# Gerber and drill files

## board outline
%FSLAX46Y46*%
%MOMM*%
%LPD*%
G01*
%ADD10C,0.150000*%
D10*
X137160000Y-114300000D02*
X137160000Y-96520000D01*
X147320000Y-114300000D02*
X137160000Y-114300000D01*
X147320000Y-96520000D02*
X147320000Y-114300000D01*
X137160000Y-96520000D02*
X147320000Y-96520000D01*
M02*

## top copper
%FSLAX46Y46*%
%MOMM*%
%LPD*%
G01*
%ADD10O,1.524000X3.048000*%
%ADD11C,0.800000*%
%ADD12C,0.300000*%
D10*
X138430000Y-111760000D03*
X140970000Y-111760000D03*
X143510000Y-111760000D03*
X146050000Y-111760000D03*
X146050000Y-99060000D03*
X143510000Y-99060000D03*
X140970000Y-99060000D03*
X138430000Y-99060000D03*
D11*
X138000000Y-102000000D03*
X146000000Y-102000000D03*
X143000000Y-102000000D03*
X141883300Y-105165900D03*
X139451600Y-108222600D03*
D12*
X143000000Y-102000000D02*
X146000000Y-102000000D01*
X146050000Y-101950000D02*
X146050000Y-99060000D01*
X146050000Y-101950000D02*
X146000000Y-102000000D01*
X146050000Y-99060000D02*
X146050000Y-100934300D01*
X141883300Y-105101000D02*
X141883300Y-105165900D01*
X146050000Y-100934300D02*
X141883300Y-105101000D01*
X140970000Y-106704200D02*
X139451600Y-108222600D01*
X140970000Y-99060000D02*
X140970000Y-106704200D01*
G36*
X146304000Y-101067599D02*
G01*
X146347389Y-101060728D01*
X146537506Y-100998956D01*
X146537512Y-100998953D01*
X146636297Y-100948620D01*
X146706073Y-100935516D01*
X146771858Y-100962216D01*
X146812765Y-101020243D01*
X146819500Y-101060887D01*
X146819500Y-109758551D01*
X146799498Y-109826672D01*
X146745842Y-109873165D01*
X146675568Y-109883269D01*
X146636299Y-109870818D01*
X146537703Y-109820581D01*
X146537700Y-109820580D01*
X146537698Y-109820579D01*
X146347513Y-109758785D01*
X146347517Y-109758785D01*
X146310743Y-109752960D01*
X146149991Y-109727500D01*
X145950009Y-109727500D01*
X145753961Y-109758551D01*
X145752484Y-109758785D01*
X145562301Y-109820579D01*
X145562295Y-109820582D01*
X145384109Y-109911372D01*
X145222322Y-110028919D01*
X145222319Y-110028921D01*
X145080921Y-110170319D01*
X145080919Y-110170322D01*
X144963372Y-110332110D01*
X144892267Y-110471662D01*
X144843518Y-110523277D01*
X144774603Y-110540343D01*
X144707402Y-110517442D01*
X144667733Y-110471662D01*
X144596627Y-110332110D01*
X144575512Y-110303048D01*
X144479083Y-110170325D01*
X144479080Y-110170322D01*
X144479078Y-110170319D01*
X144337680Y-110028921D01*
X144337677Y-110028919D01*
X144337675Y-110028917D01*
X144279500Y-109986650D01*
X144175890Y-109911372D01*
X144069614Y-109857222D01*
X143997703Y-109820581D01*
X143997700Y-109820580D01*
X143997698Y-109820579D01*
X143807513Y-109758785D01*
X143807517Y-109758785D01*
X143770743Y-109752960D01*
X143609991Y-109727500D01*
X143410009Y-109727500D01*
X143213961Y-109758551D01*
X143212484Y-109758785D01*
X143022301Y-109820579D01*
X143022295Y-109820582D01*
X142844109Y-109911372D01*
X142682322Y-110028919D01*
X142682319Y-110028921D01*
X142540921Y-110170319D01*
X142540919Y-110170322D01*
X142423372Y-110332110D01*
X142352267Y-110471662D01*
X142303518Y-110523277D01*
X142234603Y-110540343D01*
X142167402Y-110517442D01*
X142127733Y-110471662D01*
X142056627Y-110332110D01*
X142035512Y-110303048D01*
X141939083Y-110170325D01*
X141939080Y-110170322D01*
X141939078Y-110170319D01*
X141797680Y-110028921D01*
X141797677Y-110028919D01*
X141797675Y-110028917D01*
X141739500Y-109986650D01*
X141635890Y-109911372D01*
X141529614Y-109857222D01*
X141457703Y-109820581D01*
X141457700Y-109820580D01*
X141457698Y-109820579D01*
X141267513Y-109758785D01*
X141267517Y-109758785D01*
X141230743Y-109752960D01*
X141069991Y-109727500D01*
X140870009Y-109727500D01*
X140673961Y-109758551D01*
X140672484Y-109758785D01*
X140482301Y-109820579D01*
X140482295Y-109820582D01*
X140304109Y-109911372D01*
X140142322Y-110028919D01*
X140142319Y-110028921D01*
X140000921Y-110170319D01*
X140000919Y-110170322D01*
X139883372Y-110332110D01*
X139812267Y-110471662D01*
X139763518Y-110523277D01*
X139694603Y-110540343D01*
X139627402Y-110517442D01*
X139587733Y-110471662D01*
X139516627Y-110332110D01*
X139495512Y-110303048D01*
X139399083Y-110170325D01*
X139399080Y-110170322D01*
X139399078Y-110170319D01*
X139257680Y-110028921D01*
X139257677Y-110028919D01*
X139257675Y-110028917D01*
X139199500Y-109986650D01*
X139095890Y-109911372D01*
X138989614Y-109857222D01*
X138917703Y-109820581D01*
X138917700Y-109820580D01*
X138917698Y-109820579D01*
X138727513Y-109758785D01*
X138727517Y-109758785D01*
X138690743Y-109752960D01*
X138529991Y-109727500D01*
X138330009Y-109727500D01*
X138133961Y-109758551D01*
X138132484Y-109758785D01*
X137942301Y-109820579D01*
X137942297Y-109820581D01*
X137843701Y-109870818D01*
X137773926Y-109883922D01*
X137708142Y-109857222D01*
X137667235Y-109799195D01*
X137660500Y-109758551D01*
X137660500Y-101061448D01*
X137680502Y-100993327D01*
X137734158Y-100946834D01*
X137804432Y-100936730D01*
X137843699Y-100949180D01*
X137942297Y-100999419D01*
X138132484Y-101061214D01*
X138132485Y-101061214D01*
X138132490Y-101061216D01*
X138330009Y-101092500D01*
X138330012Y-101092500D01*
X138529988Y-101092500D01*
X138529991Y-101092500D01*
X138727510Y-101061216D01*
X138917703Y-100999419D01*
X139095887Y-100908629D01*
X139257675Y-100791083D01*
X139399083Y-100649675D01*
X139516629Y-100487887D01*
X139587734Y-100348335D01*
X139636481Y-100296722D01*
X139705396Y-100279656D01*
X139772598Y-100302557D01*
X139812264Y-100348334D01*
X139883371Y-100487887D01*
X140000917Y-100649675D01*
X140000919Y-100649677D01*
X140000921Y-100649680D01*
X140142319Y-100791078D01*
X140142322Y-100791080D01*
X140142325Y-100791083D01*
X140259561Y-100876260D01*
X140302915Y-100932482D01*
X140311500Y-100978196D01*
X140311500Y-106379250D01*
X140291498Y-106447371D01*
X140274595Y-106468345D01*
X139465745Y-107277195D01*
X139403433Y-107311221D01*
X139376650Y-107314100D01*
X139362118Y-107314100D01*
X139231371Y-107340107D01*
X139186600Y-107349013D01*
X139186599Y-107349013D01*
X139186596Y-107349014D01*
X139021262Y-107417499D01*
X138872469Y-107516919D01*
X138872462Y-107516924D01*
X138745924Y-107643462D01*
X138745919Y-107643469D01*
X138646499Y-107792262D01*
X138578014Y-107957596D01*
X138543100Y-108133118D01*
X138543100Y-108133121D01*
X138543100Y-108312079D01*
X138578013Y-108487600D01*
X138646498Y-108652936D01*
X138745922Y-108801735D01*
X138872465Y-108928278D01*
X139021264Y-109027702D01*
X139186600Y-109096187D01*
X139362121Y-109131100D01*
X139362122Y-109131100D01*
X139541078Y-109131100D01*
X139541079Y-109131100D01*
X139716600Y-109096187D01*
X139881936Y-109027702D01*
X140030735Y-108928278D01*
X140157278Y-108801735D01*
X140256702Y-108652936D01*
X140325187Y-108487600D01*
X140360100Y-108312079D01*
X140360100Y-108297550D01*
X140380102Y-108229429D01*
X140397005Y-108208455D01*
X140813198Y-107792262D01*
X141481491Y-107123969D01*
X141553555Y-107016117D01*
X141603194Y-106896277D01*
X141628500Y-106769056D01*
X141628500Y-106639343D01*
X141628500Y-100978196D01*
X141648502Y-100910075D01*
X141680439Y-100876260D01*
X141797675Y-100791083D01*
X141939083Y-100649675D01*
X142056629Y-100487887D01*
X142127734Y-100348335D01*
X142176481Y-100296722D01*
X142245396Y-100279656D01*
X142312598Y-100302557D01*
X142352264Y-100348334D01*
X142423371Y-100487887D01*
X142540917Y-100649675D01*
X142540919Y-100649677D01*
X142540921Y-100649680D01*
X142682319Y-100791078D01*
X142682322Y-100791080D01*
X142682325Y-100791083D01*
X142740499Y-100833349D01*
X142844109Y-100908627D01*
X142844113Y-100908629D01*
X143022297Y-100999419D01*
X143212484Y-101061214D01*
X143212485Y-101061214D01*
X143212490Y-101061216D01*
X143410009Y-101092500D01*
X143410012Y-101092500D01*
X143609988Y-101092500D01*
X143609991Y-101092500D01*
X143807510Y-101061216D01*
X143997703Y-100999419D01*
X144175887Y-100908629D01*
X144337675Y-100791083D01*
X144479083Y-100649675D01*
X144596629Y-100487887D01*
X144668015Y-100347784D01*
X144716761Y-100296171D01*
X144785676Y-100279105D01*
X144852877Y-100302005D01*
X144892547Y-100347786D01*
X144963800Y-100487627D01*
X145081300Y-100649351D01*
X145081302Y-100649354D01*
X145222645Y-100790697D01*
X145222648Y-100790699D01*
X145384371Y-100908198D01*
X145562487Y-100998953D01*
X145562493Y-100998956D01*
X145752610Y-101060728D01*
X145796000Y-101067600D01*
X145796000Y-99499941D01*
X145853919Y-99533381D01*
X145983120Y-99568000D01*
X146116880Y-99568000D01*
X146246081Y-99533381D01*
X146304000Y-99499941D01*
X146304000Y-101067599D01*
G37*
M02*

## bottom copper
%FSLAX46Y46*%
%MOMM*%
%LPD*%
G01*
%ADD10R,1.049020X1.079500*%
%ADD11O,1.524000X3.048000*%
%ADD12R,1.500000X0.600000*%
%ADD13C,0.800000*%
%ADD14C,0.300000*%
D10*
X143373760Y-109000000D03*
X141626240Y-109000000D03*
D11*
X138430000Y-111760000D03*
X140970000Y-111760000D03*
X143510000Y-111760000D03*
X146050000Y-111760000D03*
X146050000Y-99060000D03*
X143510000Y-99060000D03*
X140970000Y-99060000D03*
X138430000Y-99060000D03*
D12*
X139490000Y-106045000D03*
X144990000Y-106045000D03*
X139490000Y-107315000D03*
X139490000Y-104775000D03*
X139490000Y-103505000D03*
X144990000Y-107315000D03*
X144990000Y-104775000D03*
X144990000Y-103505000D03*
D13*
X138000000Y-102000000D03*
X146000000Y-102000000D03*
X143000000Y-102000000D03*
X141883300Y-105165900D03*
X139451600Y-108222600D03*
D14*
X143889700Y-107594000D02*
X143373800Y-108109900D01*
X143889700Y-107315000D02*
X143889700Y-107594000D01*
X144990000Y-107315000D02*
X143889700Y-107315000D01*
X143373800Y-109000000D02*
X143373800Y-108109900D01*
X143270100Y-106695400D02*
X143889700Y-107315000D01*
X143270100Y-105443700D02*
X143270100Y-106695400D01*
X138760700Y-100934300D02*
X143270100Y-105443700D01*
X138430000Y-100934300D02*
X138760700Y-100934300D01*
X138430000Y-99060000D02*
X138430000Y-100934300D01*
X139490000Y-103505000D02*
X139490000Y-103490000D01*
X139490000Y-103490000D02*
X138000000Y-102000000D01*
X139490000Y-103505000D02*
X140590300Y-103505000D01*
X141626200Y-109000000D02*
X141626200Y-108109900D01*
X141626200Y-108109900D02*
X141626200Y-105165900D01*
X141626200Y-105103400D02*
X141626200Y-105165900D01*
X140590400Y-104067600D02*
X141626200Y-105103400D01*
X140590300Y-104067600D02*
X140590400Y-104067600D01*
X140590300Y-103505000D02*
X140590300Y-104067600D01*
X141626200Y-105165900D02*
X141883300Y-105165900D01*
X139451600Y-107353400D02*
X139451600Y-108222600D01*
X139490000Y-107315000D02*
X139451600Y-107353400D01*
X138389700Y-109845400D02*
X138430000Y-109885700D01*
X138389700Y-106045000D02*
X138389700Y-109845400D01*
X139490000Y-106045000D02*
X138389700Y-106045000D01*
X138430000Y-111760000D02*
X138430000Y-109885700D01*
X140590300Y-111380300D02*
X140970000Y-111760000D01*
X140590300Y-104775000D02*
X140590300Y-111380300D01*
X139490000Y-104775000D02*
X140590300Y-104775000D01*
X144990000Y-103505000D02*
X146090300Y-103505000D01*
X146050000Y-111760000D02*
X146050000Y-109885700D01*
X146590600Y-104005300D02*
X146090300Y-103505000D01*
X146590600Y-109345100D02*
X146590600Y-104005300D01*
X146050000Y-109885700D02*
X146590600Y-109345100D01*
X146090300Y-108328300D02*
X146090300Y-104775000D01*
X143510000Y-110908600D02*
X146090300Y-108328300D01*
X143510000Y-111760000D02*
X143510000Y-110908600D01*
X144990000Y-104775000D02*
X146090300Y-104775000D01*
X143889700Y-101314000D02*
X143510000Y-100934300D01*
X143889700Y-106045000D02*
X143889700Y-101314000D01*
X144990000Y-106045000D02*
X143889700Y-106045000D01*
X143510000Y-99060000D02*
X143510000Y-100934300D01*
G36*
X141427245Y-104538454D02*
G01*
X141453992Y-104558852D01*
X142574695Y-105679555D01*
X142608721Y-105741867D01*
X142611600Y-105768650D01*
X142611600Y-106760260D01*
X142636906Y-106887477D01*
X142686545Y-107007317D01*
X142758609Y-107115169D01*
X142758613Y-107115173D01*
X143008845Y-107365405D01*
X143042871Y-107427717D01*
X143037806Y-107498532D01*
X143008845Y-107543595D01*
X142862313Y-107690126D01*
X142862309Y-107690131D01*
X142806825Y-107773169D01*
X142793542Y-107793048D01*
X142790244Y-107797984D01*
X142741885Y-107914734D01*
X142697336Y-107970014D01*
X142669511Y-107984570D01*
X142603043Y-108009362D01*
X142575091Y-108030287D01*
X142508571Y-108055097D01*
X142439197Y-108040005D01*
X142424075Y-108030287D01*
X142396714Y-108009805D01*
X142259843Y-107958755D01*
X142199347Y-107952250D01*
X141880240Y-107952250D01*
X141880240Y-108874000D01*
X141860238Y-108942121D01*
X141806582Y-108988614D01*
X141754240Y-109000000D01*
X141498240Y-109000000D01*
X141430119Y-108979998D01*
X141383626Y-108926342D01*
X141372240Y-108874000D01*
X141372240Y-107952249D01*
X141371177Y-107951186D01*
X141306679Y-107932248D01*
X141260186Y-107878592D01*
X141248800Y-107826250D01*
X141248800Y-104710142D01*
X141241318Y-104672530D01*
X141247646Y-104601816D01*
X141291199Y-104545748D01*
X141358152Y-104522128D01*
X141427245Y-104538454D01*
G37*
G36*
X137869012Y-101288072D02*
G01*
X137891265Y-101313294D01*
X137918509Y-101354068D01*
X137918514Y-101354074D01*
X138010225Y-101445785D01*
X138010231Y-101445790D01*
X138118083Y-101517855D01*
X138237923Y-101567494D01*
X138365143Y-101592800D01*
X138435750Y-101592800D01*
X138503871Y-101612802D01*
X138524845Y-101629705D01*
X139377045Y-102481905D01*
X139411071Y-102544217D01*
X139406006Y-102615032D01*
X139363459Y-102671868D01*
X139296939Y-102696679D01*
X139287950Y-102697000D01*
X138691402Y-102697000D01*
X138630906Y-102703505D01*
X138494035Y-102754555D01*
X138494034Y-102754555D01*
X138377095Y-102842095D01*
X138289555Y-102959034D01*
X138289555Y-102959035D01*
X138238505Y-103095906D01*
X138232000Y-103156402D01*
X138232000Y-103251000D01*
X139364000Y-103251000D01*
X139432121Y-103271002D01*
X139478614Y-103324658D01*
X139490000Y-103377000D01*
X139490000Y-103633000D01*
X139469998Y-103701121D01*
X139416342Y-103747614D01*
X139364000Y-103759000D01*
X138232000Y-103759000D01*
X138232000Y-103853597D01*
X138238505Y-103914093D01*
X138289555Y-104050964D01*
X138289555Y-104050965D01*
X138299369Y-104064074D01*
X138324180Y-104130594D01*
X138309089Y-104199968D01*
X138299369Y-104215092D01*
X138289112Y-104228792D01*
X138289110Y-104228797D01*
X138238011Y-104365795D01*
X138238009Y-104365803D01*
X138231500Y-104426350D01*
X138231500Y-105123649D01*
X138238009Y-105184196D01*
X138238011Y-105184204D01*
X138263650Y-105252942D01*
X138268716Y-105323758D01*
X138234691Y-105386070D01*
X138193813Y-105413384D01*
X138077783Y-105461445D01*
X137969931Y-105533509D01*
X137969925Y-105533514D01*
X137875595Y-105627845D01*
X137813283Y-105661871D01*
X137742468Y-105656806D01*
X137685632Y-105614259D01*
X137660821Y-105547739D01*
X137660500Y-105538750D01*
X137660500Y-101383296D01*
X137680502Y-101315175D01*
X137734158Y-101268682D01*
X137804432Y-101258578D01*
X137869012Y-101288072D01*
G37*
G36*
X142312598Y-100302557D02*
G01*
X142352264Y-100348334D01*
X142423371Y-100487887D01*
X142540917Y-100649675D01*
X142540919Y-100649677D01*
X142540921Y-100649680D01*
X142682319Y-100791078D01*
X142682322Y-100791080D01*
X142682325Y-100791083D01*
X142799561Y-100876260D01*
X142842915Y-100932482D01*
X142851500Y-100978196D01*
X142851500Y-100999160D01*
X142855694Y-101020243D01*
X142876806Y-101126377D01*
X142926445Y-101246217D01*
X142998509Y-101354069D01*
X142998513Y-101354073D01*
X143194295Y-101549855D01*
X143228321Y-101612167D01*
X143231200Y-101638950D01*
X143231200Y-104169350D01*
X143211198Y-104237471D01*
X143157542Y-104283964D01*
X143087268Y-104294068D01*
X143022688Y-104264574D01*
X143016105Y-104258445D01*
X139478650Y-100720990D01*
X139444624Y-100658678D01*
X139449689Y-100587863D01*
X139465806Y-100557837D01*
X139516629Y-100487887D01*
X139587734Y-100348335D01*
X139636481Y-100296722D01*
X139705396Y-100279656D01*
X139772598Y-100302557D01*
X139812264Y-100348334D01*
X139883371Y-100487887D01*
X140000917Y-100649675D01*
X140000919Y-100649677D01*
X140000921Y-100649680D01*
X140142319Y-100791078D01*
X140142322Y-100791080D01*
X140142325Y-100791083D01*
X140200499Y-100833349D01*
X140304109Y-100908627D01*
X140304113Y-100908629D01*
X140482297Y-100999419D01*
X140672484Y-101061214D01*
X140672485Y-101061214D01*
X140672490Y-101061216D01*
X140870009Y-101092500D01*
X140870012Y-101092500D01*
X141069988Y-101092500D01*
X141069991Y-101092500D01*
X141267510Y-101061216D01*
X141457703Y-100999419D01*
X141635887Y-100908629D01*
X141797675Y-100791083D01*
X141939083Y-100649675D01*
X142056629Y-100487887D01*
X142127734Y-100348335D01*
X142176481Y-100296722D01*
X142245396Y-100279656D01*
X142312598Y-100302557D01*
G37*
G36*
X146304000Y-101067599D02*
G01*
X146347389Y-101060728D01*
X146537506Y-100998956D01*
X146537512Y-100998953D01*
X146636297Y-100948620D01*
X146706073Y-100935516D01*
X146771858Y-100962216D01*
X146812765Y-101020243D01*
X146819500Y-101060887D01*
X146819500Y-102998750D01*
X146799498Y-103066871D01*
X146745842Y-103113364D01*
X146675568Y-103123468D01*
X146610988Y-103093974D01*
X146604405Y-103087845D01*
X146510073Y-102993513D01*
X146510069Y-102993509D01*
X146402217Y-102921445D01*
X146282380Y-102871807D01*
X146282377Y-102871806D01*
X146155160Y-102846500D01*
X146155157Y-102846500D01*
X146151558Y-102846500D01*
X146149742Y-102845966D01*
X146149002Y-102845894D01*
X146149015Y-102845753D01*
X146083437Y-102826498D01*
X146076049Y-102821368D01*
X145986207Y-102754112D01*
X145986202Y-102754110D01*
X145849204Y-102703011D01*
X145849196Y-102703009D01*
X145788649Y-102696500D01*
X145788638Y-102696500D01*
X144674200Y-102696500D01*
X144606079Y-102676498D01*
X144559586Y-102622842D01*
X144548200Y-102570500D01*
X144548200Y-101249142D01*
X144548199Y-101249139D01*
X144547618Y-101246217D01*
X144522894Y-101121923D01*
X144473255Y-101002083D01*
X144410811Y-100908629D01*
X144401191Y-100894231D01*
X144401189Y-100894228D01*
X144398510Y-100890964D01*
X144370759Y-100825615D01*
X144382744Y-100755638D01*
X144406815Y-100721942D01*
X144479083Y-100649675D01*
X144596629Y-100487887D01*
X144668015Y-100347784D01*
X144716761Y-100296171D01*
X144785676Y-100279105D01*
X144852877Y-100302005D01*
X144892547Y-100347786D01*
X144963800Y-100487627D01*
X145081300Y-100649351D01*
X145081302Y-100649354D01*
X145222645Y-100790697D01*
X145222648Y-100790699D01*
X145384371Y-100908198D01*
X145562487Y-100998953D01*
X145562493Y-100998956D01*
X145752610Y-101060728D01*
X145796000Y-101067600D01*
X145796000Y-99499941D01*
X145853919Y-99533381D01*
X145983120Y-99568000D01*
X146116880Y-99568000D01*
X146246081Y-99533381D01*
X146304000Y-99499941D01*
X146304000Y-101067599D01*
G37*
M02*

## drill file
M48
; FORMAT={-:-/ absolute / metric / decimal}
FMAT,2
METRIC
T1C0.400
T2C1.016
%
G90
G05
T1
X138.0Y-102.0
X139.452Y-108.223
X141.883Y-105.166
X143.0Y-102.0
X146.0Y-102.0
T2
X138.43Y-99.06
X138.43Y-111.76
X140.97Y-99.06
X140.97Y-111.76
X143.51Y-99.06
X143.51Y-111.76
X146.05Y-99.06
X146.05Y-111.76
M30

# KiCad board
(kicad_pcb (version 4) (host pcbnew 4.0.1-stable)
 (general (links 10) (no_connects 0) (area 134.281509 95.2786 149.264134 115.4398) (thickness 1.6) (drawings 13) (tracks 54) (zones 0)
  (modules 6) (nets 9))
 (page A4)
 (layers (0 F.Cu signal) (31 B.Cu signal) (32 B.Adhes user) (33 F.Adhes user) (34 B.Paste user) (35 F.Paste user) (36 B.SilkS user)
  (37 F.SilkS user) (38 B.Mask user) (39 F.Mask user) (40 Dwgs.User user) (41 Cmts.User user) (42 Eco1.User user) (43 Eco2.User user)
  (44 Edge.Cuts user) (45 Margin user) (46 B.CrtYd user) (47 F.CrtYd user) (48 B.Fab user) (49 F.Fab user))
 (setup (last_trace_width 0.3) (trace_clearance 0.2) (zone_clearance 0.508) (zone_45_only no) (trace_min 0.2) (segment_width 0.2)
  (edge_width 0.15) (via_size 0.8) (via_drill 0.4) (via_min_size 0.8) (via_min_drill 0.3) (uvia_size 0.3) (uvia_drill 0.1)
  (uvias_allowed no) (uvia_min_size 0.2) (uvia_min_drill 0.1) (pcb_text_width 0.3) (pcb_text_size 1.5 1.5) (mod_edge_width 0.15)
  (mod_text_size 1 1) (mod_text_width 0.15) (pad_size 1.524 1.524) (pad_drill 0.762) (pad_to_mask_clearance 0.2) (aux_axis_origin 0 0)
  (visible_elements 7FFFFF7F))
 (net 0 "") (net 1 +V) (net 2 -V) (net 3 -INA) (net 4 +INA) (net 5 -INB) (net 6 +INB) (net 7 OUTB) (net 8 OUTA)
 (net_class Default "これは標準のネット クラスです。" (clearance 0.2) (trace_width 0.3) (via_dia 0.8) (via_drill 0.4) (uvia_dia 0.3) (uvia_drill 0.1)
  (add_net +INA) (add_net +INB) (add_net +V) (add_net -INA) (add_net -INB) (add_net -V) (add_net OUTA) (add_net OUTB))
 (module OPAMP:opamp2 (layer F.Cu) (at 144.75 107.75)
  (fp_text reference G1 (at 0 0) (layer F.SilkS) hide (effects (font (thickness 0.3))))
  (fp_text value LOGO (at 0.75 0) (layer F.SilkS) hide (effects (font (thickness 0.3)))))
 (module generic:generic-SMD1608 (layer B.Cu) (at 142.5 109 180)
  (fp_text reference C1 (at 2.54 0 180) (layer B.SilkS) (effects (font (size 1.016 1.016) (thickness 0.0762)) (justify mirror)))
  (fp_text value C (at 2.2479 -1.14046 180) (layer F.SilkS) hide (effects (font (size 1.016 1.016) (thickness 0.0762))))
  (pad 1 smd rect (at -0.87376 0 180) (size 1.04902 1.0795) (layers B.Cu B.Paste B.Mask) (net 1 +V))
  (pad 2 smd rect (at 0.87376 0 180) (size 1.04902 1.0795) (layers B.Cu B.Paste B.Mask) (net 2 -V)))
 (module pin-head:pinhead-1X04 (layer F.Cu) (at 142.24 111.76)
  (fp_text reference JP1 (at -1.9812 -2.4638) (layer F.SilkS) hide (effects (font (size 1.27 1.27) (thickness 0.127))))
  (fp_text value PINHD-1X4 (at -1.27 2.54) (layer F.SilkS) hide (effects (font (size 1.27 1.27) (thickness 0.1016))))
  (pad 1 thru_hole oval (at -3.81 0 180) (size 1.524 3.048) (drill 1.016) (layers *.Cu F.Paste F.SilkS F.Mask) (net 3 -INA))
  (pad 2 thru_hole oval (at -1.27 0 180) (size 1.524 3.048) (drill 1.016) (layers *.Cu F.Paste F.SilkS F.Mask) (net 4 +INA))
  (pad 3 thru_hole oval (at 1.27 0 180) (size 1.524 3.048) (drill 1.016) (layers *.Cu F.Paste F.SilkS F.Mask) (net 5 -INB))
  (pad 4 thru_hole oval (at 3.81 0 180) (size 1.524 3.048) (drill 1.016) (layers *.Cu F.Paste F.SilkS F.Mask) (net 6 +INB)))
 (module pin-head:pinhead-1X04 (layer F.Cu) (at 142.24 99.06 180)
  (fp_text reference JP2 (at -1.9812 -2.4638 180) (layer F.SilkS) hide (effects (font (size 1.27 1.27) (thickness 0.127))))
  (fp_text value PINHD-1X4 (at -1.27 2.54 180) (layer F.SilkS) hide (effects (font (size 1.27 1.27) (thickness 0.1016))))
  (pad 1 thru_hole oval (at -3.81 0) (size 1.524 3.048) (drill 1.016) (layers *.Cu F.Paste F.SilkS F.Mask) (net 2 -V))
  (pad 2 thru_hole oval (at -1.27 0) (size 1.524 3.048) (drill 1.016) (layers *.Cu F.Paste F.SilkS F.Mask) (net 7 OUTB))
  (pad 3 thru_hole oval (at 1.27 0) (size 1.524 3.048) (drill 1.016) (layers *.Cu F.Paste F.SilkS F.Mask) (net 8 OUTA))
  (pad 4 thru_hole oval (at 3.81 0) (size 1.524 3.048) (drill 1.016) (layers *.Cu F.Paste F.SilkS F.Mask) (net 1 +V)))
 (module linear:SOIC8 (layer B.Cu) (at 142.24 105.41 90)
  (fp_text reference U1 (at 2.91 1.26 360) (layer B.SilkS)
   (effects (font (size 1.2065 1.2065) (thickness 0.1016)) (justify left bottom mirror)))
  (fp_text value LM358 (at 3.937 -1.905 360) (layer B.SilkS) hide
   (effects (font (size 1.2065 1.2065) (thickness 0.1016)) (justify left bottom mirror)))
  (pad 2 smd rect (at -0.635 -2.75 90) (size 0.6 1.5) (layers B.Cu B.Paste B.Mask) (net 3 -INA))
  (pad 7 smd rect (at -0.635 2.75 90) (size 0.6 1.5) (layers B.Cu B.Paste B.Mask) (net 7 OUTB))
  (pad 1 smd rect (at -1.905 -2.75 90) (size 0.6 1.5) (layers B.Cu B.Paste B.Mask) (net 8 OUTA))
  (pad 3 smd rect (at 0.635 -2.75 90) (size 0.6 1.5) (layers B.Cu B.Paste B.Mask) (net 4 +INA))
  (pad 4 smd rect (at 1.905 -2.75 90) (size 0.6 1.5) (layers B.Cu B.Paste B.Mask) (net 2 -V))
  (pad 8 smd rect (at -1.905 2.75 90) (size 0.6 1.5) (layers B.Cu B.Paste B.Mask) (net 1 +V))
  (pad 6 smd rect (at 0.635 2.75 90) (size 0.6 1.5) (layers B.Cu B.Paste B.Mask) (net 5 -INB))
  (pad 5 smd rect (at 1.905 2.75 90) (size 0.6 1.5) (layers B.Cu B.Paste B.Mask) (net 6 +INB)))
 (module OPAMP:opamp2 (layer F.Cu) (at 139.75 107.75)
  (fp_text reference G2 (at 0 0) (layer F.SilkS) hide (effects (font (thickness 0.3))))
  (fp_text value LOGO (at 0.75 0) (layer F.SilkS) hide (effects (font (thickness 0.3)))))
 (gr_line (start 137.16 114.3) (end 137.16 96.52) (angle 90) (layer Edge.Cuts) (width 0.15))
 (gr_line (start 147.32 114.3) (end 137.16 114.3) (angle 90) (layer Edge.Cuts) (width 0.15))
 (gr_line (start 147.32 96.52) (end 147.32 114.3) (angle 90) (layer Edge.Cuts) (width 0.15))
 (gr_line (start 137.16 96.52) (end 147.32 96.52) (angle 90) (layer Edge.Cuts) (width 0.15))
 (segment (start 143.8897 107.594) (end 143.3738 108.1099) (width 0.3) (layer B.Cu) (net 1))
 (segment (start 143.8897 107.315) (end 143.8897 107.594) (width 0.3) (layer B.Cu) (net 1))
 (segment (start 144.99 107.315) (end 143.8897 107.315) (width 0.3) (layer B.Cu) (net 1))
 (segment (start 143.3738 109) (end 143.3738 108.1099) (width 0.3) (layer B.Cu) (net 1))
 (segment (start 143.2701 106.6954) (end 143.8897 107.315) (width 0.3) (layer B.Cu) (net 1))
 (segment (start 143.2701 105.4437) (end 143.2701 106.6954) (width 0.3) (layer B.Cu) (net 1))
 (segment (start 138.7607 100.9343) (end 143.2701 105.4437) (width 0.3) (layer B.Cu) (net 1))
 (segment (start 138.43 100.9343) (end 138.7607 100.9343) (width 0.3) (layer B.Cu) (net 1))
 (segment (start 138.43 99.06) (end 138.43 100.9343) (width 0.3) (layer B.Cu) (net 1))
 (segment (start 139.49 103.505) (end 139.49 103.49) (width 0.3) (layer B.Cu) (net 2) (status C00000))
 (segment (start 139.49 103.49) (end 138 102) (width 0.3) (layer B.Cu) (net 2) (status 400000))
 (via (at 138 102) (size 0.8) (drill 0.4) (layers F.Cu B.Cu) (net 2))
 (segment (start 143 102) (end 146 102) (width 0.3) (layer F.Cu) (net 2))
 (segment (start 146.05 101.95) (end 146.05 99.06) (width 0.3) (layer F.Cu) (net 2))
 (via (at 146 102) (size 0.8) (drill 0.4) (layers F.Cu B.Cu) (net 2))
 (segment (start 146.05 101.95) (end 146 102) (width 0.3) (layer F.Cu) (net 2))
 (via (at 143 102) (size 0.8) (drill 0.4) (layers F.Cu B.Cu) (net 2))
 (via (at 141.8833 105.1659) (size 0.8) (layers F.Cu B.Cu) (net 2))
 (segment (start 139.49 103.505) (end 140.5903 103.505) (width 0.3) (layer B.Cu) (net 2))
 (segment (start 146.05 99.06) (end 146.05 100.9343) (width 0.3) (layer F.Cu) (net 2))
 (segment (start 141.8833 105.101) (end 141.8833 105.1659) (width 0.3) (layer F.Cu) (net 2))
 (segment (start 146.05 100.9343) (end 141.8833 105.101) (width 0.3) (layer F.Cu) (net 2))
 (segment (start 141.6262 109) (end 141.6262 108.1099) (width 0.3) (layer B.Cu) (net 2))
 (segment (start 141.6262 108.1099) (end 141.6262 105.1659) (width 0.3) (layer B.Cu) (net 2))
 (segment (start 141.6262 105.1034) (end 141.6262 105.1659) (width 0.3) (layer B.Cu) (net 2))
 (segment (start 140.5904 104.0676) (end 141.6262 105.1034) (width 0.3) (layer B.Cu) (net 2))
 (segment (start 140.5903 104.0676) (end 140.5904 104.0676) (width 0.3) (layer B.Cu) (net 2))
 (segment (start 140.5903 103.505) (end 140.5903 104.0676) (width 0.3) (layer B.Cu) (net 2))
 (segment (start 141.6262 105.1659) (end 141.8833 105.1659) (width 0.3) (layer B.Cu) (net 2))
 (via (at 139.4516 108.2226) (size 0.8) (layers F.Cu B.Cu) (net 8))
 (segment (start 139.4516 107.3534) (end 139.4516 108.2226) (width 0.3) (layer B.Cu) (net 8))
 (segment (start 139.49 107.315) (end 139.4516 107.3534) (width 0.3) (layer B.Cu) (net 8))
 (segment (start 140.97 106.7042) (end 139.4516 108.2226) (width 0.3) (layer F.Cu) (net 8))
 (segment (start 140.97 99.06) (end 140.97 106.7042) (width 0.3) (layer F.Cu) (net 8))
 (segment (start 138.3897 109.8454) (end 138.43 109.8857) (width 0.3) (layer B.Cu) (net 3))
 (segment (start 138.3897 106.045) (end 138.3897 109.8454) (width 0.3) (layer B.Cu) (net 3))
 (segment (start 139.49 106.045) (end 138.3897 106.045) (width 0.3) (layer B.Cu) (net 3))
 (segment (start 138.43 111.76) (end 138.43 109.8857) (width 0.3) (layer B.Cu) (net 3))
 (segment (start 140.5903 111.3803) (end 140.97 111.76) (width 0.3) (layer B.Cu) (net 4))
 (segment (start 140.5903 104.775) (end 140.5903 111.3803) (width 0.3) (layer B.Cu) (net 4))
 (segment (start 139.49 104.775) (end 140.5903 104.775) (width 0.3) (layer B.Cu) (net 4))
 (segment (start 144.99 103.505) (end 146.0903 103.505) (width 0.3) (layer B.Cu) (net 6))
 (segment (start 146.05 111.76) (end 146.05 109.8857) (width 0.3) (layer B.Cu) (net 6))
 (segment (start 146.5906 104.0053) (end 146.0903 103.505) (width 0.3) (layer B.Cu) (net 6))
 (segment (start 146.5906 109.3451) (end 146.5906 104.0053) (width 0.3) (layer B.Cu) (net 6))
 (segment (start 146.05 109.8857) (end 146.5906 109.3451) (width 0.3) (layer B.Cu) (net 6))
 (segment (start 146.0903 108.3283) (end 146.0903 104.775) (width 0.3) (layer B.Cu) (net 5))
 (segment (start 143.51 110.9086) (end 146.0903 108.3283) (width 0.3) (layer B.Cu) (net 5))
 (segment (start 143.51 111.76) (end 143.51 110.9086) (width 0.3) (layer B.Cu) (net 5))
 (segment (start 144.99 104.775) (end 146.0903 104.775) (width 0.3) (layer B.Cu) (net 5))
 (segment (start 143.8897 101.314) (end 143.51 100.9343) (width 0.3) (layer B.Cu) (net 7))
 (segment (start 143.8897 106.045) (end 143.8897 101.314) (width 0.3) (layer B.Cu) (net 7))
 (segment (start 144.99 106.045) (end 143.8897 106.045) (width 0.3) (layer B.Cu) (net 7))
 (segment (start 143.51 99.06) (end 143.51 100.9343) (width 0.3) (layer B.Cu) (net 7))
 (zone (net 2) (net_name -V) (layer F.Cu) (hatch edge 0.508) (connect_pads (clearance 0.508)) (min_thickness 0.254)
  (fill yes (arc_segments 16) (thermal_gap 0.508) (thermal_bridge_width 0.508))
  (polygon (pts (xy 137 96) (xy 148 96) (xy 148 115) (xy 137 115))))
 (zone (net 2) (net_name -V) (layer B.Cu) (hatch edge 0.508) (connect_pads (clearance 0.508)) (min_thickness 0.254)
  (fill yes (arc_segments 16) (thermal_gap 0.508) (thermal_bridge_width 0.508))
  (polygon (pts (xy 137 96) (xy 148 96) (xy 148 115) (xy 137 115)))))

